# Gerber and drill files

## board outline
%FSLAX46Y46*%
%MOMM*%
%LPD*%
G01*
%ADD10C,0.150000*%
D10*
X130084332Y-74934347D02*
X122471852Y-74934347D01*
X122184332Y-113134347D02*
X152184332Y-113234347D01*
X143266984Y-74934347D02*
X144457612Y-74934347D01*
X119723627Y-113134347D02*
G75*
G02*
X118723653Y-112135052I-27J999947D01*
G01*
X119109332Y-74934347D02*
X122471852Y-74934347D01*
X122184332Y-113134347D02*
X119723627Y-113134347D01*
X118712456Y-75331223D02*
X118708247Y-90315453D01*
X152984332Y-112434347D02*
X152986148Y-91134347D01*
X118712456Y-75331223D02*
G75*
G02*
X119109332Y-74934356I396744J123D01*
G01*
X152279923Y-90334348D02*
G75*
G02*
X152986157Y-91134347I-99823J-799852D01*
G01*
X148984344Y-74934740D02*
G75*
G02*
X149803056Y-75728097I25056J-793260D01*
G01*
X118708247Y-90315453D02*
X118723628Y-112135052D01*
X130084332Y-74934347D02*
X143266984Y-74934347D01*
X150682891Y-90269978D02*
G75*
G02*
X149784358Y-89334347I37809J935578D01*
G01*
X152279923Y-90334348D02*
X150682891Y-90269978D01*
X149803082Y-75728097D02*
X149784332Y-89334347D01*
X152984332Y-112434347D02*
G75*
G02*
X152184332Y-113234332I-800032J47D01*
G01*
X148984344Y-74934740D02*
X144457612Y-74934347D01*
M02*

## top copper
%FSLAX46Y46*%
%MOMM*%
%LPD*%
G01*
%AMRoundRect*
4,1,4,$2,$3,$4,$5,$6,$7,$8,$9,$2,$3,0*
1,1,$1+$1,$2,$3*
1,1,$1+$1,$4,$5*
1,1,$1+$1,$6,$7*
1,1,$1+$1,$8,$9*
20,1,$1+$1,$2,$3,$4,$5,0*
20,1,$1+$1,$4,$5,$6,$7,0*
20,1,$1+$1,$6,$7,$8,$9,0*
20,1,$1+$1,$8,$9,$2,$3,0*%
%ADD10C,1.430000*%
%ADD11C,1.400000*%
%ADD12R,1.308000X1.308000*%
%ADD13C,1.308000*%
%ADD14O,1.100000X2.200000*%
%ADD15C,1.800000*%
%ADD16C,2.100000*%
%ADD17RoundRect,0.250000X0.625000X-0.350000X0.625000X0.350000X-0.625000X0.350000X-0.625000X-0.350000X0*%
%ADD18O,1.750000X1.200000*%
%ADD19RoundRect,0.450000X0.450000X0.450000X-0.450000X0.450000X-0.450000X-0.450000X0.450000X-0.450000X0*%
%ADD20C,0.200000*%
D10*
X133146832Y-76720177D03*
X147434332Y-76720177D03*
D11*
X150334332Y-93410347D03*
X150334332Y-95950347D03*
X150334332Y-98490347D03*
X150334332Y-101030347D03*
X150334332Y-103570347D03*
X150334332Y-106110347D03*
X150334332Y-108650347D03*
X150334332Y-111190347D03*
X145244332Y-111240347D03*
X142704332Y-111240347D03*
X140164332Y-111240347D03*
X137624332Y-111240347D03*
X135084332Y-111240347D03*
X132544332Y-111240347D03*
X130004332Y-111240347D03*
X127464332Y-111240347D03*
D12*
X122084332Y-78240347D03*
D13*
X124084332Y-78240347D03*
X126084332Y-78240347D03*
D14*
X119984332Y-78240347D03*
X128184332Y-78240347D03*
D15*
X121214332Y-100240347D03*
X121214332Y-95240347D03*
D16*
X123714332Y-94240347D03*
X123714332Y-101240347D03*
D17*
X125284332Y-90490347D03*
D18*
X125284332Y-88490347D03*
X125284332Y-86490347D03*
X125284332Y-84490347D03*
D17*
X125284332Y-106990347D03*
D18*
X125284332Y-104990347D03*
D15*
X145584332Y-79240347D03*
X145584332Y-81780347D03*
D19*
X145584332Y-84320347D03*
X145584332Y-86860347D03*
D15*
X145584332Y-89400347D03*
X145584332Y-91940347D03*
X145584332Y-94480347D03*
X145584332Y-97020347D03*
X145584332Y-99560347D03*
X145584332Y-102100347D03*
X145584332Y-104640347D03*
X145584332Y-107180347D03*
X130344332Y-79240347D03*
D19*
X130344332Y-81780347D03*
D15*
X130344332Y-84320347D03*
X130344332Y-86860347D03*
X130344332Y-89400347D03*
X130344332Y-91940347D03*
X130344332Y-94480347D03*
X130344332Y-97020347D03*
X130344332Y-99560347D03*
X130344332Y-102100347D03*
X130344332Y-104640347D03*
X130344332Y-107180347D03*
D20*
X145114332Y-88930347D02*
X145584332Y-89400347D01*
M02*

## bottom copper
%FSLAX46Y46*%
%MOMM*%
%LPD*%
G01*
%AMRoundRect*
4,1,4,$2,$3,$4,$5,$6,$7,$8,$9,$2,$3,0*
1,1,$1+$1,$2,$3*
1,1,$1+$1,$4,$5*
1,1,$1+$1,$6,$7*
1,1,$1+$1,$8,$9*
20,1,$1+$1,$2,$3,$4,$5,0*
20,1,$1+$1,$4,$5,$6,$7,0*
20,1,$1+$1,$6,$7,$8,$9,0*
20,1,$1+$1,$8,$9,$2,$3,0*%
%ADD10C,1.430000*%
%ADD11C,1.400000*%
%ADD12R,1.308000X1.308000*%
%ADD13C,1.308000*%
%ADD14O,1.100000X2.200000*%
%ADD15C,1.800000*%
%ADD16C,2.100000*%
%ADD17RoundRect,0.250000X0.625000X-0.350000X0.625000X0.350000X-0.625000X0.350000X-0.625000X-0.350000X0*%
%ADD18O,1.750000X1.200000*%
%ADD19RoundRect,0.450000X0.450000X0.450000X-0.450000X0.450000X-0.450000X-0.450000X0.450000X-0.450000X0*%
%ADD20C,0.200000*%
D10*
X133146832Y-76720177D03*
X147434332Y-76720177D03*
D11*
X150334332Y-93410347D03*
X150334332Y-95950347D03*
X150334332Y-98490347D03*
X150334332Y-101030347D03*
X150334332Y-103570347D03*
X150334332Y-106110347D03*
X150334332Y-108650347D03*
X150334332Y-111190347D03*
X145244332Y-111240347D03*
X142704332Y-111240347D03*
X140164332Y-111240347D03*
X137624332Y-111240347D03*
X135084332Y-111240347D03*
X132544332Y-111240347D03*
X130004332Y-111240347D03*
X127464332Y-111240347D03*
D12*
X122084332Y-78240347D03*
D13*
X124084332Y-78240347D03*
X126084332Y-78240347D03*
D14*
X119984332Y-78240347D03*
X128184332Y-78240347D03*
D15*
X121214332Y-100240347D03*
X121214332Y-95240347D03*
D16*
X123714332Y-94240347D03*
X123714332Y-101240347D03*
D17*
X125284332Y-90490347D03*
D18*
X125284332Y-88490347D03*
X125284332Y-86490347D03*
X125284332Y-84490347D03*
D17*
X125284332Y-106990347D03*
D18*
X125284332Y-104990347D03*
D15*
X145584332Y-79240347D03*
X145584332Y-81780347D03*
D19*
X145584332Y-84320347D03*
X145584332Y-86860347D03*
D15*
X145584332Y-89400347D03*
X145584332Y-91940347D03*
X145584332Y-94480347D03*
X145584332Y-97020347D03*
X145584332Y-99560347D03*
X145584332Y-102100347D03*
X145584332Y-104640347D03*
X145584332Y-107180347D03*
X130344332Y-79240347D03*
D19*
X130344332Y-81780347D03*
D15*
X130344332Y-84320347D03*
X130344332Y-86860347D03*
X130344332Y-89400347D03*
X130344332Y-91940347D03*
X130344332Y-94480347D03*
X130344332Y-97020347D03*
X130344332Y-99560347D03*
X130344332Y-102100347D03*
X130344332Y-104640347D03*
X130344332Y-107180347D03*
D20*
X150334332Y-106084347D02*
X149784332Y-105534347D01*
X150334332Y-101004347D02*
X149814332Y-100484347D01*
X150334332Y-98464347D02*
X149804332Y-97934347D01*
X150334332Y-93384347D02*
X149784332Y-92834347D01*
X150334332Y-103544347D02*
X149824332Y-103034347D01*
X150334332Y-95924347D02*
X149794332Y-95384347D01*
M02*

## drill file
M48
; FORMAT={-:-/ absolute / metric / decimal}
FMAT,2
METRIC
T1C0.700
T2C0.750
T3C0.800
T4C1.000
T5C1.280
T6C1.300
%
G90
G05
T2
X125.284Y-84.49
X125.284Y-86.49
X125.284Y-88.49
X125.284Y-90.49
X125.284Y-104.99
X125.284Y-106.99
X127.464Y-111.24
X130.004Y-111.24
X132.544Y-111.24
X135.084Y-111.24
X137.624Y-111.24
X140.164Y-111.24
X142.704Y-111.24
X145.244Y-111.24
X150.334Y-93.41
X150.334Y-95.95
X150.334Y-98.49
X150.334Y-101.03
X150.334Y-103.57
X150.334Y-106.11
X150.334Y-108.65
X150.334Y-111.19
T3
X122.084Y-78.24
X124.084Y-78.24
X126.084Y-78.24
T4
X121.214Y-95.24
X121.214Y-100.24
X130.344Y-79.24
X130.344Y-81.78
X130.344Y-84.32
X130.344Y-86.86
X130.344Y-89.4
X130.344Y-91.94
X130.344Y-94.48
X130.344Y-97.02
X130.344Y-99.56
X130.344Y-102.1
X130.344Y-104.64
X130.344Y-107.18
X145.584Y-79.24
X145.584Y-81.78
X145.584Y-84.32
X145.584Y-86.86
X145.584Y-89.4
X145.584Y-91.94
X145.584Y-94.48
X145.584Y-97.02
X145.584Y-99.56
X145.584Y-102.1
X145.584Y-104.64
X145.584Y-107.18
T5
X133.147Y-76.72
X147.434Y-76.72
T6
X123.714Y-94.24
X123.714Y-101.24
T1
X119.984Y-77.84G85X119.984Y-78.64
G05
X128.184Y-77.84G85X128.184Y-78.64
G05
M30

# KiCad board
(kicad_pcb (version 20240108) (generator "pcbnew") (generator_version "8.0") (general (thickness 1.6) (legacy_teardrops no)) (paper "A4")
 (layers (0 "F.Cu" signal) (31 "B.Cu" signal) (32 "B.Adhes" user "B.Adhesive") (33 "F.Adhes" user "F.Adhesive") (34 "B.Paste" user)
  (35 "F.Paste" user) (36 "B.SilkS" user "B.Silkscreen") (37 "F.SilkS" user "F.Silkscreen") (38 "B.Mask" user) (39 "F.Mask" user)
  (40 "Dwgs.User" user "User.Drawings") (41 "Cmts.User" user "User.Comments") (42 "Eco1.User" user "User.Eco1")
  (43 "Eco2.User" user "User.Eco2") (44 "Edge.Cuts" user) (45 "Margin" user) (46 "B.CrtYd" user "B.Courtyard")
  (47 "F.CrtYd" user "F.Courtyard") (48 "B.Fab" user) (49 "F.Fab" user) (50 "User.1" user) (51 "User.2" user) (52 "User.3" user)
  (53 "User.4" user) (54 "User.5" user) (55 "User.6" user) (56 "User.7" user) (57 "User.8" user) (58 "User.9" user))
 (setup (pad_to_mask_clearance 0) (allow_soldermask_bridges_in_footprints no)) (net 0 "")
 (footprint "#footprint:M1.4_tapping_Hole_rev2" (layer "F.Cu") (at 133.146832 76.720177)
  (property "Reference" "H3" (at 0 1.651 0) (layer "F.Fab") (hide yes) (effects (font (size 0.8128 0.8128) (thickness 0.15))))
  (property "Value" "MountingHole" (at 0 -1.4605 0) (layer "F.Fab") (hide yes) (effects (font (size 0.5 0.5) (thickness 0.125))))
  (pad "" thru_hole circle (at 0 0) (size 1.43 1.43) (drill 1.28) (layers "*.Cu" "*.Mask") (remove_unused_layers no)))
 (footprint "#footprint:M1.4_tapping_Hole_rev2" (layer "F.Cu") (at 147.434332 76.720177)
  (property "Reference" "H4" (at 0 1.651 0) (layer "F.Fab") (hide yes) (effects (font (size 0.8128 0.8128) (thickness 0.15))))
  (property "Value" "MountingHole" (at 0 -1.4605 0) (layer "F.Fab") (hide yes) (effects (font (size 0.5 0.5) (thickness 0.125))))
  (pad "" thru_hole circle (at 0 0) (size 1.43 1.43) (drill 1.28) (layers "*.Cu" "*.Mask") (remove_unused_layers no)))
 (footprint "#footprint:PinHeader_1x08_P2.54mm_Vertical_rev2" (layer "B.Cu") (at 150.334332 93.410347 180)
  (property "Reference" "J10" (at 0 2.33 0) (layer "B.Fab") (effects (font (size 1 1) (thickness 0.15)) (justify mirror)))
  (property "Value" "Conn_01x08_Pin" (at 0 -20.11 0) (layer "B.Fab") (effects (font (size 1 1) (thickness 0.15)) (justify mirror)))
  (pad "1" thru_hole circle (at 0 0 180) (size 1.4 1.4) (drill 0.75) (layers "*.Cu" "*.Mask") (remove_unused_layers no))
  (pad "2" thru_hole circle (at 0 -2.54 180) (size 1.4 1.4) (drill 0.75) (layers "*.Cu" "*.Mask") (remove_unused_layers no))
  (pad "3" thru_hole circle (at 0 -5.08 180) (size 1.4 1.4) (drill 0.75) (layers "*.Cu" "*.Mask") (remove_unused_layers no))
  (pad "4" thru_hole circle (at 0 -7.62 180) (size 1.4 1.4) (drill 0.75) (layers "*.Cu" "*.Mask") (remove_unused_layers no))
  (pad "5" thru_hole circle (at 0 -10.16 180) (size 1.4 1.4) (drill 0.75) (layers "*.Cu" "*.Mask") (remove_unused_layers no))
  (pad "6" thru_hole circle (at 0 -12.7 180) (size 1.4 1.4) (drill 0.75) (layers "*.Cu" "*.Mask") (remove_unused_layers no))
  (pad "7" thru_hole circle (at 0 -15.24 180) (size 1.4 1.4) (drill 0.75) (layers "*.Cu" "*.Mask") (remove_unused_layers no))
  (pad "8" thru_hole circle (at 0 -17.78 180) (size 1.4 1.4) (drill 0.75) (layers "*.Cu" "*.Mask") (remove_unused_layers no)))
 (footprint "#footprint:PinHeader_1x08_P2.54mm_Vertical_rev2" (layer "B.Cu") (at 145.244332 111.240347 90)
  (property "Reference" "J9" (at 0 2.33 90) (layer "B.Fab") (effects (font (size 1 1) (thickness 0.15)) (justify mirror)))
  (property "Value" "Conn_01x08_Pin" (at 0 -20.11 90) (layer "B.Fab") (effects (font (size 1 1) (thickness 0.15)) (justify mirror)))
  (pad "1" thru_hole circle (at 0 0 90) (size 1.4 1.4) (drill 0.75) (layers "*.Cu" "*.Mask") (remove_unused_layers no))
  (pad "2" thru_hole circle (at 0 -2.54 90) (size 1.4 1.4) (drill 0.75) (layers "*.Cu" "*.Mask") (remove_unused_layers no))
  (pad "3" thru_hole circle (at 0 -5.08 90) (size 1.4 1.4) (drill 0.75) (layers "*.Cu" "*.Mask") (remove_unused_layers no))
  (pad "4" thru_hole circle (at 0 -7.62 90) (size 1.4 1.4) (drill 0.75) (layers "*.Cu" "*.Mask") (remove_unused_layers no))
  (pad "5" thru_hole circle (at 0 -10.16 90) (size 1.4 1.4) (drill 0.75) (layers "*.Cu" "*.Mask") (remove_unused_layers no))
  (pad "6" thru_hole circle (at 0 -12.7 90) (size 1.4 1.4) (drill 0.75) (layers "*.Cu" "*.Mask") (remove_unused_layers no))
  (pad "7" thru_hole circle (at 0 -15.24 90) (size 1.4 1.4) (drill 0.75) (layers "*.Cu" "*.Mask") (remove_unused_layers no))
  (pad "8" thru_hole circle (at 0 -17.78 90) (size 1.4 1.4) (drill 0.75) (layers "*.Cu" "*.Mask") (remove_unused_layers no)))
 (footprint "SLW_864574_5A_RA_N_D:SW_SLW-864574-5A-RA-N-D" (layer "B.Cu") (at 124.084332 78.240347)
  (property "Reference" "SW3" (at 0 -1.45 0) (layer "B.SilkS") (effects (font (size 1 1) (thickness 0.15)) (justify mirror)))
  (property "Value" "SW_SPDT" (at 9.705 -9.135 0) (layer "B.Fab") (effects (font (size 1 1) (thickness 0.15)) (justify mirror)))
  (pad "1" thru_hole rect (at -2 0) (size 1.308 1.308) (drill 0.8) (layers "*.Cu" "*.Mask") (remove_unused_layers no)
   (solder_mask_margin 0.102))
  (pad "2" thru_hole circle (at 0 0) (size 1.308 1.308) (drill 0.8) (layers "*.Cu" "*.Mask") (remove_unused_layers no)
   (solder_mask_margin 0.102))
  (pad "3" thru_hole circle (at 2 0) (size 1.308 1.308) (drill 0.8) (layers "*.Cu" "*.Mask") (remove_unused_layers no)
   (solder_mask_margin 0.102))
  (pad "SH1" thru_hole oval (at -4.1 0) (size 1.1 2.2) (drill oval 0.7 1.5) (layers "*.Cu" "*.Mask") (remove_unused_layers no)
   (solder_mask_margin 0.102))
  (pad "SH2" thru_hole oval (at 4.1 0) (size 1.1 2.2) (drill oval 0.7 1.5) (layers "*.Cu" "*.Mask") (remove_unused_layers no)
   (solder_mask_margin 0.102)))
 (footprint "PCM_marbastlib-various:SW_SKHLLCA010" (layer "B.Cu") (at 122.464332 97.740347 -90)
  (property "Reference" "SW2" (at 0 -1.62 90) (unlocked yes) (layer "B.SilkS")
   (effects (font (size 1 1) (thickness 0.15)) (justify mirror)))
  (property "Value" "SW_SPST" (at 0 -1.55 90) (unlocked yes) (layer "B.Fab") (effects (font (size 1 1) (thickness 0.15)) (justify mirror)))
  (pad "1" thru_hole circle (at 2.5 1.25 270) (size 1.8 1.8) (drill 1) (layers "*.Cu" "F.Mask") (remove_unused_layers no))
  (pad "2" thru_hole circle (at -2.5 1.25 270) (size 1.8 1.8) (drill 1) (layers "*.Cu" "F.Mask") (remove_unused_layers no))
  (pad "MP" thru_hole circle (at -3.5 -1.25 270) (size 2.1 2.1) (drill 1.3) (layers "*.Cu" "*.Mask") (remove_unused_layers no))
  (pad "MP" thru_hole circle (at 3.5 -1.25 270) (size 2.1 2.1) (drill 1.3) (layers "*.Cu" "*.Mask") (remove_unused_layers no)))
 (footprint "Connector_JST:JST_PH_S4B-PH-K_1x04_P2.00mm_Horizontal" (layer "B.Cu") (at 125.284332 90.490347 90)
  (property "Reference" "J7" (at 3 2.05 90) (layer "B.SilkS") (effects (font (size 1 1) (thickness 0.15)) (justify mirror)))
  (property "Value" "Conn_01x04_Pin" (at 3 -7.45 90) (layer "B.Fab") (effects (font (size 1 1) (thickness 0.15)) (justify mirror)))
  (pad "1" thru_hole roundrect (at 0 0 90) (size 1.2 1.75) (drill 0.75) (layers "*.Cu" "*.Mask") (remove_unused_layers no)
   (roundrect_rratio 0.208333))
  (pad "2" thru_hole oval (at 2 0 90) (size 1.2 1.75) (drill 0.75) (layers "*.Cu" "*.Mask") (remove_unused_layers no))
  (pad "3" thru_hole oval (at 4 0 90) (size 1.2 1.75) (drill 0.75) (layers "*.Cu" "*.Mask") (remove_unused_layers no))
  (pad "4" thru_hole oval (at 6 0 90) (size 1.2 1.75) (drill 0.75) (layers "*.Cu" "*.Mask") (remove_unused_layers no)))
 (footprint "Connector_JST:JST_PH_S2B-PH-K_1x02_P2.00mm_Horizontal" (layer "B.Cu") (at 125.284332 106.990347 90)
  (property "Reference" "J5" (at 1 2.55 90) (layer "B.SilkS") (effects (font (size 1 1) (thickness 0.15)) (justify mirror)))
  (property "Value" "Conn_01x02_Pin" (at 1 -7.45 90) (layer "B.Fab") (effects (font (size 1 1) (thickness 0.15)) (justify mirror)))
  (pad "1" thru_hole roundrect (at 0 0 90) (size 1.2 1.75) (drill 0.75) (layers "*.Cu" "*.Mask") (remove_unused_layers no)
   (roundrect_rratio 0.208333))
  (pad "2" thru_hole oval (at 2 0 90) (size 1.2 1.75) (drill 0.75) (layers "*.Cu" "*.Mask") (remove_unused_layers no)))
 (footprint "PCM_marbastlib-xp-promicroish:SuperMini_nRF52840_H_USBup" (layer "B.Cu") (at 137.964332 93.210347 180)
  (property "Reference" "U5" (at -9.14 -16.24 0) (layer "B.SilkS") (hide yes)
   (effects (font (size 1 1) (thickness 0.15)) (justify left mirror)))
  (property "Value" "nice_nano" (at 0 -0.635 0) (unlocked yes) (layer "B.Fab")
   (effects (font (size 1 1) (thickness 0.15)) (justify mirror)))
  (pad "1" thru_hole circle (at -7.62 13.97 180) (size 1.8 1.8) (drill 1) (layers "*.Cu" "F.Mask") (remove_unused_layers no))
  (pad "2" thru_hole circle (at -7.62 11.43 180) (size 1.8 1.8) (drill 1) (layers "*.Cu" "F.Mask") (remove_unused_layers no))
  (pad "3" thru_hole roundrect (at -7.62 8.89 180) (size 1.8 1.8) (drill 1) (layers "*.Cu" "F.Mask") (remove_unused_layers no)
   (roundrect_rratio 0.25))
  (pad "4" thru_hole roundrect (at -7.62 6.35 180) (size 1.8 1.8) (drill 1) (layers "*.Cu" "F.Mask") (remove_unused_layers no)
   (roundrect_rratio 0.25))
  (pad "5" thru_hole circle (at -7.62 3.81 180) (size 1.8 1.8) (drill 1) (layers "*.Cu" "F.Mask") (remove_unused_layers no))
  (pad "6" thru_hole circle (at -7.62 1.27 180) (size 1.8 1.8) (drill 1) (layers "*.Cu" "F.Mask") (remove_unused_layers no))
  (pad "7" thru_hole circle (at -7.62 -1.27 180) (size 1.8 1.8) (drill 1) (layers "*.Cu" "F.Mask") (remove_unused_layers no))
  (pad "8" thru_hole circle (at -7.62 -3.81 180) (size 1.8 1.8) (drill 1) (layers "*.Cu" "F.Mask") (remove_unused_layers no))
  (pad "9" thru_hole circle (at -7.62 -6.35 180) (size 1.8 1.8) (drill 1) (layers "*.Cu" "F.Mask") (remove_unused_layers no))
  (pad "10" thru_hole circle (at -7.62 -8.89 180) (size 1.8 1.8) (drill 1) (layers "*.Cu" "F.Mask") (remove_unused_layers no))
  (pad "11" thru_hole circle (at -7.62 -11.43 180) (size 1.8 1.8) (drill 1) (layers "*.Cu" "F.Mask") (remove_unused_layers no))
  (pad "12" thru_hole circle (at -7.62 -13.97 180) (size 1.8 1.8) (drill 1) (layers "*.Cu" "F.Mask") (remove_unused_layers no))
  (pad "13" thru_hole circle (at 7.62 13.97 180) (size 1.8 1.8) (drill 1) (layers "*.Cu" "F.Mask") (remove_unused_layers no))
  (pad "14" thru_hole roundrect (at 7.62 11.43 180) (size 1.8 1.8) (drill 1) (layers "*.Cu" "F.Mask") (remove_unused_layers no)
   (roundrect_rratio 0.25))
  (pad "15" thru_hole circle (at 7.62 8.89 180) (size 1.8 1.8) (drill 1) (layers "*.Cu" "F.Mask") (remove_unused_layers no))
  (pad "16" thru_hole circle (at 7.62 6.35 180) (size 1.8 1.8) (drill 1) (layers "*.Cu" "F.Mask") (remove_unused_layers no))
  (pad "17" thru_hole circle (at 7.62 3.81 180) (size 1.8 1.8) (drill 1) (layers "*.Cu" "F.Mask") (remove_unused_layers no))
  (pad "18" thru_hole circle (at 7.62 1.27 180) (size 1.8 1.8) (drill 1) (layers "*.Cu" "F.Mask") (remove_unused_layers no))
  (pad "19" thru_hole circle (at 7.62 -1.27 180) (size 1.8 1.8) (drill 1) (layers "*.Cu" "F.Mask") (remove_unused_layers no))
  (pad "20" thru_hole circle (at 7.62 -3.81 180) (size 1.8 1.8) (drill 1) (layers "*.Cu" "F.Mask") (remove_unused_layers no))
  (pad "21" thru_hole circle (at 7.62 -6.35 180) (size 1.8 1.8) (drill 1) (layers "*.Cu" "F.Mask") (remove_unused_layers no))
  (pad "22" thru_hole circle (at 7.62 -8.89 180) (size 1.8 1.8) (drill 1) (layers "*.Cu" "F.Mask") (remove_unused_layers no))
  (pad "23" thru_hole circle (at 7.62 -11.43 180) (size 1.8 1.8) (drill 1) (layers "*.Cu" "F.Mask") (remove_unused_layers no))
  (pad "24" thru_hole circle (at 7.62 -13.97 180) (size 1.8 1.8) (drill 1) (layers "*.Cu" "F.Mask") (remove_unused_layers no))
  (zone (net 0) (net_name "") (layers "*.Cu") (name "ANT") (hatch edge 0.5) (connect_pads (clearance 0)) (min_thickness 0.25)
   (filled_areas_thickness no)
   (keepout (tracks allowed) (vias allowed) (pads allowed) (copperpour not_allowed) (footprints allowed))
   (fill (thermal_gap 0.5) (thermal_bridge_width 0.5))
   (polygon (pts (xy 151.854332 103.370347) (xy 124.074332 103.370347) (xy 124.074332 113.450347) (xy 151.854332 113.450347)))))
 (gr_line (start 130.084332 74.934347) (end 122.471852 74.934347) (stroke (width 0.15) (type solid)) (layer "Edge.Cuts"))
 (gr_line (start 122.184332 113.134347) (end 152.184332 113.234347) (stroke (width 0.15) (type default)) (layer "Edge.Cuts"))
 (gr_line (start 143.266984 74.934347) (end 144.457612 74.934347) (stroke (width 0.15) (type solid)) (layer "Edge.Cuts"))
 (gr_arc (start 119.723627 113.134347) (mid 119.016761 112.841712) (end 118.723628 112.135052) (stroke (width 0.15) (type default))
  (layer "Edge.Cuts"))
 (gr_line (start 119.109332 74.934347) (end 122.471852 74.934347) (stroke (width 0.15) (type solid)) (layer "Edge.Cuts"))
 (gr_line (start 122.184332 113.134347) (end 119.723627 113.134347) (stroke (width 0.15) (type default)) (layer "Edge.Cuts"))
 (gr_line (start 118.712456 75.331223) (end 118.708247 90.315453) (stroke (width 0.15) (type solid)) (layer "Edge.Cuts"))
 (gr_line (start 152.984332 112.434347) (end 152.986148 91.134347) (stroke (width 0.15) (type default)) (layer "Edge.Cuts"))
 (gr_arc (start 118.712456 75.331223) (mid 118.828656 75.050547) (end 119.109332 74.934347) (stroke (width 0.15) (type solid))
  (layer "Edge.Cuts"))
 (gr_arc (start 152.279923 90.334348) (mid 152.784371 90.600752) (end 152.986148 91.134347) (stroke (width 0.15) (type default))
  (layer "Edge.Cuts"))
 (gr_arc (start 148.984344 74.93474) (mid 149.561724 75.158033) (end 149.803082 75.728097) (stroke (width 0.15) (type solid))
  (layer "Edge.Cuts"))
 (gr_line (start 118.708247 90.315453) (end 118.723628 112.135052) (stroke (width 0.15) (type default)) (layer "Edge.Cuts"))
 (gr_line (start 130.084332 74.934347) (end 143.266984 74.934347) (stroke (width 0.15) (type solid)) (layer "Edge.Cuts"))
 (gr_arc (start 150.682891 90.269978) (mid 150.045341 89.982973) (end 149.784332 89.334347) (stroke (width 0.15) (type default))
  (layer "Edge.Cuts"))
 (gr_line (start 152.279923 90.334348) (end 150.682891 90.269978) (stroke (width 0.15) (type default)) (layer "Edge.Cuts"))
 (gr_line (start 149.803082 75.728097) (end 149.784332 89.334347) (stroke (width 0.15) (type default)) (layer "Edge.Cuts"))
 (gr_arc (start 152.984332 112.434347) (mid 152.750014 113.000029) (end 152.184332 113.234347) (stroke (width 0.15) (type default))
  (layer "Edge.Cuts"))
 (gr_line (start 148.984344 74.93474) (end 144.457612 74.934347) (stroke (width 0.15) (type solid)) (layer "Edge.Cuts"))
 (segment (start 145.114332 88.930347) (end 145.584332 89.400347) (width 0.2) (layer "F.Cu") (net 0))
 (segment (start 150.334332 106.084347) (end 149.784332 105.534347) (width 0.2) (layer "B.Cu") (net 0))
 (segment (start 150.334332 101.004347) (end 149.814332 100.484347) (width 0.2) (layer "B.Cu") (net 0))
 (segment (start 150.334332 98.464347) (end 149.804332 97.934347) (width 0.2) (layer "B.Cu") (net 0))
 (segment (start 150.334332 93.384347) (end 149.784332 92.834347) (width 0.2) (layer "B.Cu") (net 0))
 (segment (start 150.334332 103.544347) (end 149.824332 103.034347) (width 0.2) (layer "B.Cu") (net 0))
 (segment (start 150.334332 95.924347) (end 149.794332 95.384347) (width 0.2) (layer "B.Cu") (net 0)))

